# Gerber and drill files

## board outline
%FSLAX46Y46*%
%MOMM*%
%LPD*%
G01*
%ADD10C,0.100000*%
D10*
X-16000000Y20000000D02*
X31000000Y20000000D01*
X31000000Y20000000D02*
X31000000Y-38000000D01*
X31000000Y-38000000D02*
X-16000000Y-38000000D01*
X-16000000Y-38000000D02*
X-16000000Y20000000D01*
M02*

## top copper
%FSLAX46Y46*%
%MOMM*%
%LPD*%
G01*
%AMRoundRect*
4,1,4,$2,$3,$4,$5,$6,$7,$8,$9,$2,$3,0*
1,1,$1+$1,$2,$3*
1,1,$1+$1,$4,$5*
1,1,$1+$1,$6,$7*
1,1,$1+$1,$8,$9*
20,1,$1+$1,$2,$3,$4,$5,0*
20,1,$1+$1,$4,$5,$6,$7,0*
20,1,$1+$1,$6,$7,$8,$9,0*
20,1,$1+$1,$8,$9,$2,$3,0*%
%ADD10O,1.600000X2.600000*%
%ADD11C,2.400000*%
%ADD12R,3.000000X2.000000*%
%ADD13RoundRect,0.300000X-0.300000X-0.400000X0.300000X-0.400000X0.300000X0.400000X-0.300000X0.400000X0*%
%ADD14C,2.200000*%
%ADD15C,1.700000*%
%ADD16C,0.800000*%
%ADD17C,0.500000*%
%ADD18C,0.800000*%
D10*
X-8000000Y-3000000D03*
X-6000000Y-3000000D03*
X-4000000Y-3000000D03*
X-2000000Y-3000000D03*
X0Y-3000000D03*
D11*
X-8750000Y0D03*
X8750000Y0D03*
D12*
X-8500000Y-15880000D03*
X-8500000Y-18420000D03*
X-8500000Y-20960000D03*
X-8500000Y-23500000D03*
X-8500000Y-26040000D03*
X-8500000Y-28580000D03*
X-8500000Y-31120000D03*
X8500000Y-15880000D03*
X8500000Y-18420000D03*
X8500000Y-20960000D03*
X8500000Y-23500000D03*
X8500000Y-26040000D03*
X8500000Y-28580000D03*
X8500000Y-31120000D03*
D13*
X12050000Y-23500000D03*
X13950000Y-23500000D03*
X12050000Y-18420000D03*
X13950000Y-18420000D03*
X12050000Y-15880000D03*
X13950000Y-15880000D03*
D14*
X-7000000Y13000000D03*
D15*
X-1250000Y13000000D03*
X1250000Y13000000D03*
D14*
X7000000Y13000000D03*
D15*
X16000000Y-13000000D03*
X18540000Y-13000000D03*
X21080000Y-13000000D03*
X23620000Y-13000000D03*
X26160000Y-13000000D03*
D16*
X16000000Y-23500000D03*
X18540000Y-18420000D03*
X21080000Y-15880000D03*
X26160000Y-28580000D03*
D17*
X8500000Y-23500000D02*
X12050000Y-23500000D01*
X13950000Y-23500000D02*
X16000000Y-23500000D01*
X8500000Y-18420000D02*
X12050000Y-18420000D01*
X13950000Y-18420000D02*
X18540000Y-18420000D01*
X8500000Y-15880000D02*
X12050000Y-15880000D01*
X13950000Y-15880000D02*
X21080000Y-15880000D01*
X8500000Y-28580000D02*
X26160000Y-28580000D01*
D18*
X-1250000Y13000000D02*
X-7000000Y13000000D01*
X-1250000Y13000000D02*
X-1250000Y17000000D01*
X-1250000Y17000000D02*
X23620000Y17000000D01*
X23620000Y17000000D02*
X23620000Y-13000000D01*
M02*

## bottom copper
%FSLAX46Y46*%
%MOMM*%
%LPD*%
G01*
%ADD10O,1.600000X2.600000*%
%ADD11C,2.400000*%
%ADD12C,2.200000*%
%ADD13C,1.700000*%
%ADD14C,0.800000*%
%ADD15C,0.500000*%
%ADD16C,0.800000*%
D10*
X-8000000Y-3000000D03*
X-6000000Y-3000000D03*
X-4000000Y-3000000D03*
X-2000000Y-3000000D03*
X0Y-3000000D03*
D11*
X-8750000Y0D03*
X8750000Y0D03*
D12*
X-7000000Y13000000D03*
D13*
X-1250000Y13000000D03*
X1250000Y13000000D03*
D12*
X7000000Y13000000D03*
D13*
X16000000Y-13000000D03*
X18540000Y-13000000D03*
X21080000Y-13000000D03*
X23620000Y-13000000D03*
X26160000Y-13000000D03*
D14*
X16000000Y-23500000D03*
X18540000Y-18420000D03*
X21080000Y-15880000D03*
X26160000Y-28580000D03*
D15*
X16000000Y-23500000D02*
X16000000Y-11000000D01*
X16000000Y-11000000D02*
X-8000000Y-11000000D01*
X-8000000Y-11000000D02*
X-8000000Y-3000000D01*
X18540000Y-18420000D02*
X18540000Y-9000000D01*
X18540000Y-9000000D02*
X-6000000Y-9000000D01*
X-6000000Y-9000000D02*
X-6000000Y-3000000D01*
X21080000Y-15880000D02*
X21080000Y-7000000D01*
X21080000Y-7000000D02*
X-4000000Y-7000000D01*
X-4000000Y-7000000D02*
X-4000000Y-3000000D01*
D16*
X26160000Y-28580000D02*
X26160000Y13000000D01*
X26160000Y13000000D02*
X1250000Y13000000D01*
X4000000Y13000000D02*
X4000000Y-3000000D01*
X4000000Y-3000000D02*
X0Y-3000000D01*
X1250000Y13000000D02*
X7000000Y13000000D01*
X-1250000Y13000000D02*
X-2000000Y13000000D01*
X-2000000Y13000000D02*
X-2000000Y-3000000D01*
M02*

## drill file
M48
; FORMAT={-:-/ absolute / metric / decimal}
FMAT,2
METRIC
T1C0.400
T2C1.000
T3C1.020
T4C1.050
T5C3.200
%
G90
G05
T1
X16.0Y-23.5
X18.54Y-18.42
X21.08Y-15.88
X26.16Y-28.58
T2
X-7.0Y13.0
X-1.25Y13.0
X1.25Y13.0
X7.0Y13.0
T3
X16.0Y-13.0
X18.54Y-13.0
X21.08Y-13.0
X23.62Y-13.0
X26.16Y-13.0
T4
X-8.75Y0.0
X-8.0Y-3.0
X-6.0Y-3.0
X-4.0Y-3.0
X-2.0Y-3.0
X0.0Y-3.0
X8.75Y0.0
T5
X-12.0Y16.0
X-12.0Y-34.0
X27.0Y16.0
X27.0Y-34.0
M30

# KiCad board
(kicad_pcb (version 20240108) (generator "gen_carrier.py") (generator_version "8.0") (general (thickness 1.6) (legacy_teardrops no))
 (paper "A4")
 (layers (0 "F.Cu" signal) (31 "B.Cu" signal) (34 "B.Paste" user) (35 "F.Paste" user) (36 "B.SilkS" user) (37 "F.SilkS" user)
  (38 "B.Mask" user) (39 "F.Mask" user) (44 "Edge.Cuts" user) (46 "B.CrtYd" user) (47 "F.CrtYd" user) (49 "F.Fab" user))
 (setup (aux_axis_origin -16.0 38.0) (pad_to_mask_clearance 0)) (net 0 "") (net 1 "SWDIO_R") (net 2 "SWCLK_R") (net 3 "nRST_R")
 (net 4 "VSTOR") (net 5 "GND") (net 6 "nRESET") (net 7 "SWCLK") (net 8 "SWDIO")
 (gr_line (start -16.0 -20.0) (end 31.0 -20.0) (stroke (width 0.1) (type default)) (layer "Edge.Cuts"))
 (gr_line (start 31.0 -20.0) (end 31.0 38.0) (stroke (width 0.1) (type default)) (layer "Edge.Cuts"))
 (gr_line (start 31.0 38.0) (end -16.0 38.0) (stroke (width 0.1) (type default)) (layer "Edge.Cuts"))
 (gr_line (start -16.0 38.0) (end -16.0 -20.0) (stroke (width 0.1) (type default)) (layer "Edge.Cuts"))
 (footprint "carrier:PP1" (layer "F.Cu") (at -8.0 3.0)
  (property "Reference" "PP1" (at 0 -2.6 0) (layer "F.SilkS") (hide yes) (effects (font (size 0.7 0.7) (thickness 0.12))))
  (pad "1" thru_hole oval (at 0 0) (size 1.6 2.6) (drill 1.05) (layers "*.Cu" "*.Mask") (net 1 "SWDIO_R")))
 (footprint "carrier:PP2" (layer "F.Cu") (at -6.0 3.0)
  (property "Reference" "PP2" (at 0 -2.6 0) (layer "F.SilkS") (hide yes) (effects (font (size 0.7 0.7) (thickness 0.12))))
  (pad "1" thru_hole oval (at 0 0) (size 1.6 2.6) (drill 1.05) (layers "*.Cu" "*.Mask") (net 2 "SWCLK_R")))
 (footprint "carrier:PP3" (layer "F.Cu") (at -4.0 3.0)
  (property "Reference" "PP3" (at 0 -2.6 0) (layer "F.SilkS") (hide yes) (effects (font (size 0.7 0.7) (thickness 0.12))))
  (pad "1" thru_hole oval (at 0 0) (size 1.6 2.6) (drill 1.05) (layers "*.Cu" "*.Mask") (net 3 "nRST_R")))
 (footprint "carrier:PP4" (layer "F.Cu") (at -2.0 3.0)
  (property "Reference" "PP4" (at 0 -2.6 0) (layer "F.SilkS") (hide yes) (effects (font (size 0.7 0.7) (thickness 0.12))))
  (pad "1" thru_hole oval (at 0 0) (size 1.6 2.6) (drill 1.05) (layers "*.Cu" "*.Mask") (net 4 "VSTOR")))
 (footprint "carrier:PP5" (layer "F.Cu") (at 0.0 3.0)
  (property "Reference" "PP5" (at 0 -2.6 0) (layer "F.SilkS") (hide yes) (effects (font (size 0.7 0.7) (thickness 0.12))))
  (pad "1" thru_hole oval (at 0 0) (size 1.6 2.6) (drill 1.05) (layers "*.Cu" "*.Mask") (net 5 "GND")))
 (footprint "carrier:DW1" (layer "F.Cu") (at -8.75 0.0)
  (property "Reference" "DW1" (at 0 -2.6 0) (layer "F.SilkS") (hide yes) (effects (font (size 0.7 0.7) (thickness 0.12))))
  (pad "1" thru_hole circle (at 0 0) (size 2.4 2.4) (drill 1.05) (layers "*.Cu" "*.Mask")))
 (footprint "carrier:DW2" (layer "F.Cu") (at 8.75 0.0)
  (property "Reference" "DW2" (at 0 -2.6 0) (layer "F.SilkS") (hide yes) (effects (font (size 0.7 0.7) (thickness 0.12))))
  (pad "1" thru_hole circle (at 0 0) (size 2.4 2.4) (drill 1.05) (layers "*.Cu" "*.Mask")))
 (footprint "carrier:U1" (layer "F.Cu") (at 0 0)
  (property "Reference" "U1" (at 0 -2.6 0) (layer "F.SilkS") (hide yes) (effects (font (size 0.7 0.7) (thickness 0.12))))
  (pad "1" smd rect (at -8.5 15.879999999999999) (size 3.0 2.0) (layers "F.Cu" "F.Paste" "F.Mask"))
  (pad "2" smd rect (at -8.5 18.419999999999998) (size 3.0 2.0) (layers "F.Cu" "F.Paste" "F.Mask"))
  (pad "3" smd rect (at -8.5 20.96) (size 3.0 2.0) (layers "F.Cu" "F.Paste" "F.Mask"))
  (pad "4" smd rect (at -8.5 23.5) (size 3.0 2.0) (layers "F.Cu" "F.Paste" "F.Mask"))
  (pad "5" smd rect (at -8.5 26.04) (size 3.0 2.0) (layers "F.Cu" "F.Paste" "F.Mask"))
  (pad "6" smd rect (at -8.5 28.58) (size 3.0 2.0) (layers "F.Cu" "F.Paste" "F.Mask"))
  (pad "7" smd rect (at -8.5 31.119999999999997) (size 3.0 2.0) (layers "F.Cu" "F.Paste" "F.Mask"))
  (pad "8" smd rect (at 8.5 15.879999999999999) (size 3.0 2.0) (layers "F.Cu" "F.Paste" "F.Mask") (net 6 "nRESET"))
  (pad "9" smd rect (at 8.5 18.419999999999998) (size 3.0 2.0) (layers "F.Cu" "F.Paste" "F.Mask") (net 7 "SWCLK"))
  (pad "10" smd rect (at 8.5 20.96) (size 3.0 2.0) (layers "F.Cu" "F.Paste" "F.Mask"))
  (pad "11" smd rect (at 8.5 23.5) (size 3.0 2.0) (layers "F.Cu" "F.Paste" "F.Mask") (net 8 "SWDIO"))
  (pad "12" smd rect (at 8.5 26.04) (size 3.0 2.0) (layers "F.Cu" "F.Paste" "F.Mask"))
  (pad "13" smd rect (at 8.5 28.58) (size 3.0 2.0) (layers "F.Cu" "F.Paste" "F.Mask") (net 5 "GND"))
  (pad "14" smd rect (at 8.5 31.119999999999997) (size 3.0 2.0) (layers "F.Cu" "F.Paste" "F.Mask")))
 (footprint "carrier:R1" (layer "F.Cu") (at 13.0 23.5)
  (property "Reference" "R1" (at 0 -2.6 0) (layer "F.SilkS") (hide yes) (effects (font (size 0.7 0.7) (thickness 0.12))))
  (pad "1" smd roundrect (at -0.95 0) (size 1.2 1.4) (layers "F.Cu" "F.Paste" "F.Mask") (roundrect_rratio 0.25) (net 8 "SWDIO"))
  (pad "2" smd roundrect (at 0.95 0) (size 1.2 1.4) (layers "F.Cu" "F.Paste" "F.Mask") (roundrect_rratio 0.25) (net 1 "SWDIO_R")))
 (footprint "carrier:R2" (layer "F.Cu") (at 13.0 18.419999999999998)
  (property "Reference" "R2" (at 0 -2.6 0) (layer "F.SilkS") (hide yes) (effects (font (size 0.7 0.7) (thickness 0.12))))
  (pad "1" smd roundrect (at -0.95 0) (size 1.2 1.4) (layers "F.Cu" "F.Paste" "F.Mask") (roundrect_rratio 0.25) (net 7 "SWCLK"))
  (pad "2" smd roundrect (at 0.95 0) (size 1.2 1.4) (layers "F.Cu" "F.Paste" "F.Mask") (roundrect_rratio 0.25) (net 2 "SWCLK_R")))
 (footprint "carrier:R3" (layer "F.Cu") (at 13.0 15.879999999999999)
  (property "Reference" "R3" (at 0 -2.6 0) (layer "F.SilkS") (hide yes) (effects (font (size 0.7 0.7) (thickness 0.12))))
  (pad "1" smd roundrect (at -0.95 0) (size 1.2 1.4) (layers "F.Cu" "F.Paste" "F.Mask") (roundrect_rratio 0.25) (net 6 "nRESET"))
  (pad "2" smd roundrect (at 0.95 0) (size 1.2 1.4) (layers "F.Cu" "F.Paste" "F.Mask") (roundrect_rratio 0.25) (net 3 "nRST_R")))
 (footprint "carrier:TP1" (layer "F.Cu") (at -7.0 -13.0)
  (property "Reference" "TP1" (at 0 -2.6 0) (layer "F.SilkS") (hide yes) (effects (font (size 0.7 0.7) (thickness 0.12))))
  (pad "1" thru_hole circle (at 0 0) (size 2.2 2.2) (drill 1.0) (layers "*.Cu" "*.Mask") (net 4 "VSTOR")))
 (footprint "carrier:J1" (layer "F.Cu") (at 0.0 -13.0)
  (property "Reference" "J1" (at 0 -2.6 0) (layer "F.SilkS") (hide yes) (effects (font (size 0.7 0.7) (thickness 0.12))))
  (pad "1" thru_hole circle (at -1.25 0) (size 1.7 1.7) (drill 1.0) (layers "*.Cu" "*.Mask") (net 4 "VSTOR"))
  (pad "2" thru_hole circle (at 1.25 0) (size 1.7 1.7) (drill 1.0) (layers "*.Cu" "*.Mask") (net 5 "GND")))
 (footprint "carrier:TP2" (layer "F.Cu") (at 7.0 -13.0)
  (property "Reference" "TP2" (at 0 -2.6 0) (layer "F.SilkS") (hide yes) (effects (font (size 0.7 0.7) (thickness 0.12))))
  (pad "1" thru_hole circle (at 0 0) (size 2.2 2.2) (drill 1.0) (layers "*.Cu" "*.Mask") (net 5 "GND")))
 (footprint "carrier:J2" (layer "F.Cu") (at 0.0 13.0)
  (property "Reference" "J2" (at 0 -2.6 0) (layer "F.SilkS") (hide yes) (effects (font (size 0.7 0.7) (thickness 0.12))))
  (pad "1" thru_hole circle (at 16.0 0) (size 1.7 1.7) (drill 1.02) (layers "*.Cu" "*.Mask") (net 1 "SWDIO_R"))
  (pad "2" thru_hole circle (at 18.54 0) (size 1.7 1.7) (drill 1.02) (layers "*.Cu" "*.Mask") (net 2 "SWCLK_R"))
  (pad "3" thru_hole circle (at 21.08 0) (size 1.7 1.7) (drill 1.02) (layers "*.Cu" "*.Mask") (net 3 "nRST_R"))
  (pad "4" thru_hole circle (at 23.62 0) (size 1.7 1.7) (drill 1.02) (layers "*.Cu" "*.Mask") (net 4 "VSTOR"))
  (pad "5" thru_hole circle (at 26.16 0) (size 1.7 1.7) (drill 1.02) (layers "*.Cu" "*.Mask") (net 5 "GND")))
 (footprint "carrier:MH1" (layer "F.Cu") (at -12.0 -16.0)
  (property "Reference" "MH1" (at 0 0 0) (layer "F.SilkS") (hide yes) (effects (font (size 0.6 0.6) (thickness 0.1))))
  (pad "" np_thru_hole circle (at 0 0) (size 3.2 3.2) (drill 3.2) (layers "F&B.Cu" "*.Mask")))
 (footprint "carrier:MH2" (layer "F.Cu") (at 27.0 -16.0)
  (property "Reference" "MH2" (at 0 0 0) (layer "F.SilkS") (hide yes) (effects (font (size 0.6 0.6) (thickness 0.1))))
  (pad "" np_thru_hole circle (at 0 0) (size 3.2 3.2) (drill 3.2) (layers "F&B.Cu" "*.Mask")))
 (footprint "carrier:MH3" (layer "F.Cu") (at -12.0 34.0)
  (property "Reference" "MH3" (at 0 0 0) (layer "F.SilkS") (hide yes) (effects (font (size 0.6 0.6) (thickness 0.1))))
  (pad "" np_thru_hole circle (at 0 0) (size 3.2 3.2) (drill 3.2) (layers "F&B.Cu" "*.Mask")))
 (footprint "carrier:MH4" (layer "F.Cu") (at 27.0 34.0)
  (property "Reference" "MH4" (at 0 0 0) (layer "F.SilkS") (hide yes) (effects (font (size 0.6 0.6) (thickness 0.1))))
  (pad "" np_thru_hole circle (at 0 0) (size 3.2 3.2) (drill 3.2) (layers "F&B.Cu" "*.Mask")))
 (via (at 16.0 23.5) (size 0.8) (drill 0.4) (layers "F.Cu" "B.Cu") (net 1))
 (via (at 18.54 18.419999999999998) (size 0.8) (drill 0.4) (layers "F.Cu" "B.Cu") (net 2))
 (via (at 21.08 15.879999999999999) (size 0.8) (drill 0.4) (layers "F.Cu" "B.Cu") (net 3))
 (via (at 26.16 28.58) (size 0.8) (drill 0.4) (layers "F.Cu" "B.Cu") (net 5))
 (segment (start 8.5 23.5) (end 12.05 23.5) (width 0.5) (layer "F.Cu") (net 8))
 (segment (start 13.95 23.5) (end 16.0 23.5) (width 0.5) (layer "F.Cu") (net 1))
 (segment (start 16.0 23.5) (end 16.0 11.0) (width 0.5) (layer "B.Cu") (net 1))
 (segment (start 16.0 11.0) (end -8.0 11.0) (width 0.5) (layer "B.Cu") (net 1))
 (segment (start -8.0 11.0) (end -8.0 3.0) (width 0.5) (layer "B.Cu") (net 1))
 (segment (start 8.5 18.42) (end 12.05 18.42) (width 0.5) (layer "F.Cu") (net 7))
 (segment (start 13.95 18.42) (end 18.54 18.42) (width 0.5) (layer "F.Cu") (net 2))
 (segment (start 18.54 18.42) (end 18.54 9.0) (width 0.5) (layer "B.Cu") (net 2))
 (segment (start 18.54 9.0) (end -6.0 9.0) (width 0.5) (layer "B.Cu") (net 2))
 (segment (start -6.0 9.0) (end -6.0 3.0) (width 0.5) (layer "B.Cu") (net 2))
 (segment (start 8.5 15.88) (end 12.05 15.88) (width 0.5) (layer "F.Cu") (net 6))
 (segment (start 13.95 15.88) (end 21.08 15.88) (width 0.5) (layer "F.Cu") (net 3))
 (segment (start 21.08 15.88) (end 21.08 7.0) (width 0.5) (layer "B.Cu") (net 3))
 (segment (start 21.08 7.0) (end -4.0 7.0) (width 0.5) (layer "B.Cu") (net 3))
 (segment (start -4.0 7.0) (end -4.0 3.0) (width 0.5) (layer "B.Cu") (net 3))
 (segment (start 8.5 28.58) (end 26.16 28.58) (width 0.5) (layer "F.Cu") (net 5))
 (segment (start 26.16 28.58) (end 26.16 -13.0) (width 0.8) (layer "B.Cu") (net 5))
 (segment (start 26.16 -13.0) (end 1.25 -13.0) (width 0.8) (layer "B.Cu") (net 5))
 (segment (start 4.0 -13.0) (end 4.0 3.0) (width 0.8) (layer "B.Cu") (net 5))
 (segment (start 4.0 3.0) (end 0.0 3.0) (width 0.8) (layer "B.Cu") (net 5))
 (segment (start 1.25 -13.0) (end 7.0 -13.0) (width 0.8) (layer "B.Cu") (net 5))
 (segment (start -1.25 -13.0) (end -2.0 -13.0) (width 0.8) (layer "B.Cu") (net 4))
 (segment (start -2.0 -13.0) (end -2.0 3.0) (width 0.8) (layer "B.Cu") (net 4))
 (segment (start -1.25 -13.0) (end -7.0 -13.0) (width 0.8) (layer "F.Cu") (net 4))
 (segment (start -1.25 -13.0) (end -1.25 -17.0) (width 0.8) (layer "F.Cu") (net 4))
 (segment (start -1.25 -17.0) (end 23.62 -17.0) (width 0.8) (layer "F.Cu") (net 4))
 (segment (start 23.62 -17.0) (end 23.62 13.0) (width 0.8) (layer "F.Cu") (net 4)))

